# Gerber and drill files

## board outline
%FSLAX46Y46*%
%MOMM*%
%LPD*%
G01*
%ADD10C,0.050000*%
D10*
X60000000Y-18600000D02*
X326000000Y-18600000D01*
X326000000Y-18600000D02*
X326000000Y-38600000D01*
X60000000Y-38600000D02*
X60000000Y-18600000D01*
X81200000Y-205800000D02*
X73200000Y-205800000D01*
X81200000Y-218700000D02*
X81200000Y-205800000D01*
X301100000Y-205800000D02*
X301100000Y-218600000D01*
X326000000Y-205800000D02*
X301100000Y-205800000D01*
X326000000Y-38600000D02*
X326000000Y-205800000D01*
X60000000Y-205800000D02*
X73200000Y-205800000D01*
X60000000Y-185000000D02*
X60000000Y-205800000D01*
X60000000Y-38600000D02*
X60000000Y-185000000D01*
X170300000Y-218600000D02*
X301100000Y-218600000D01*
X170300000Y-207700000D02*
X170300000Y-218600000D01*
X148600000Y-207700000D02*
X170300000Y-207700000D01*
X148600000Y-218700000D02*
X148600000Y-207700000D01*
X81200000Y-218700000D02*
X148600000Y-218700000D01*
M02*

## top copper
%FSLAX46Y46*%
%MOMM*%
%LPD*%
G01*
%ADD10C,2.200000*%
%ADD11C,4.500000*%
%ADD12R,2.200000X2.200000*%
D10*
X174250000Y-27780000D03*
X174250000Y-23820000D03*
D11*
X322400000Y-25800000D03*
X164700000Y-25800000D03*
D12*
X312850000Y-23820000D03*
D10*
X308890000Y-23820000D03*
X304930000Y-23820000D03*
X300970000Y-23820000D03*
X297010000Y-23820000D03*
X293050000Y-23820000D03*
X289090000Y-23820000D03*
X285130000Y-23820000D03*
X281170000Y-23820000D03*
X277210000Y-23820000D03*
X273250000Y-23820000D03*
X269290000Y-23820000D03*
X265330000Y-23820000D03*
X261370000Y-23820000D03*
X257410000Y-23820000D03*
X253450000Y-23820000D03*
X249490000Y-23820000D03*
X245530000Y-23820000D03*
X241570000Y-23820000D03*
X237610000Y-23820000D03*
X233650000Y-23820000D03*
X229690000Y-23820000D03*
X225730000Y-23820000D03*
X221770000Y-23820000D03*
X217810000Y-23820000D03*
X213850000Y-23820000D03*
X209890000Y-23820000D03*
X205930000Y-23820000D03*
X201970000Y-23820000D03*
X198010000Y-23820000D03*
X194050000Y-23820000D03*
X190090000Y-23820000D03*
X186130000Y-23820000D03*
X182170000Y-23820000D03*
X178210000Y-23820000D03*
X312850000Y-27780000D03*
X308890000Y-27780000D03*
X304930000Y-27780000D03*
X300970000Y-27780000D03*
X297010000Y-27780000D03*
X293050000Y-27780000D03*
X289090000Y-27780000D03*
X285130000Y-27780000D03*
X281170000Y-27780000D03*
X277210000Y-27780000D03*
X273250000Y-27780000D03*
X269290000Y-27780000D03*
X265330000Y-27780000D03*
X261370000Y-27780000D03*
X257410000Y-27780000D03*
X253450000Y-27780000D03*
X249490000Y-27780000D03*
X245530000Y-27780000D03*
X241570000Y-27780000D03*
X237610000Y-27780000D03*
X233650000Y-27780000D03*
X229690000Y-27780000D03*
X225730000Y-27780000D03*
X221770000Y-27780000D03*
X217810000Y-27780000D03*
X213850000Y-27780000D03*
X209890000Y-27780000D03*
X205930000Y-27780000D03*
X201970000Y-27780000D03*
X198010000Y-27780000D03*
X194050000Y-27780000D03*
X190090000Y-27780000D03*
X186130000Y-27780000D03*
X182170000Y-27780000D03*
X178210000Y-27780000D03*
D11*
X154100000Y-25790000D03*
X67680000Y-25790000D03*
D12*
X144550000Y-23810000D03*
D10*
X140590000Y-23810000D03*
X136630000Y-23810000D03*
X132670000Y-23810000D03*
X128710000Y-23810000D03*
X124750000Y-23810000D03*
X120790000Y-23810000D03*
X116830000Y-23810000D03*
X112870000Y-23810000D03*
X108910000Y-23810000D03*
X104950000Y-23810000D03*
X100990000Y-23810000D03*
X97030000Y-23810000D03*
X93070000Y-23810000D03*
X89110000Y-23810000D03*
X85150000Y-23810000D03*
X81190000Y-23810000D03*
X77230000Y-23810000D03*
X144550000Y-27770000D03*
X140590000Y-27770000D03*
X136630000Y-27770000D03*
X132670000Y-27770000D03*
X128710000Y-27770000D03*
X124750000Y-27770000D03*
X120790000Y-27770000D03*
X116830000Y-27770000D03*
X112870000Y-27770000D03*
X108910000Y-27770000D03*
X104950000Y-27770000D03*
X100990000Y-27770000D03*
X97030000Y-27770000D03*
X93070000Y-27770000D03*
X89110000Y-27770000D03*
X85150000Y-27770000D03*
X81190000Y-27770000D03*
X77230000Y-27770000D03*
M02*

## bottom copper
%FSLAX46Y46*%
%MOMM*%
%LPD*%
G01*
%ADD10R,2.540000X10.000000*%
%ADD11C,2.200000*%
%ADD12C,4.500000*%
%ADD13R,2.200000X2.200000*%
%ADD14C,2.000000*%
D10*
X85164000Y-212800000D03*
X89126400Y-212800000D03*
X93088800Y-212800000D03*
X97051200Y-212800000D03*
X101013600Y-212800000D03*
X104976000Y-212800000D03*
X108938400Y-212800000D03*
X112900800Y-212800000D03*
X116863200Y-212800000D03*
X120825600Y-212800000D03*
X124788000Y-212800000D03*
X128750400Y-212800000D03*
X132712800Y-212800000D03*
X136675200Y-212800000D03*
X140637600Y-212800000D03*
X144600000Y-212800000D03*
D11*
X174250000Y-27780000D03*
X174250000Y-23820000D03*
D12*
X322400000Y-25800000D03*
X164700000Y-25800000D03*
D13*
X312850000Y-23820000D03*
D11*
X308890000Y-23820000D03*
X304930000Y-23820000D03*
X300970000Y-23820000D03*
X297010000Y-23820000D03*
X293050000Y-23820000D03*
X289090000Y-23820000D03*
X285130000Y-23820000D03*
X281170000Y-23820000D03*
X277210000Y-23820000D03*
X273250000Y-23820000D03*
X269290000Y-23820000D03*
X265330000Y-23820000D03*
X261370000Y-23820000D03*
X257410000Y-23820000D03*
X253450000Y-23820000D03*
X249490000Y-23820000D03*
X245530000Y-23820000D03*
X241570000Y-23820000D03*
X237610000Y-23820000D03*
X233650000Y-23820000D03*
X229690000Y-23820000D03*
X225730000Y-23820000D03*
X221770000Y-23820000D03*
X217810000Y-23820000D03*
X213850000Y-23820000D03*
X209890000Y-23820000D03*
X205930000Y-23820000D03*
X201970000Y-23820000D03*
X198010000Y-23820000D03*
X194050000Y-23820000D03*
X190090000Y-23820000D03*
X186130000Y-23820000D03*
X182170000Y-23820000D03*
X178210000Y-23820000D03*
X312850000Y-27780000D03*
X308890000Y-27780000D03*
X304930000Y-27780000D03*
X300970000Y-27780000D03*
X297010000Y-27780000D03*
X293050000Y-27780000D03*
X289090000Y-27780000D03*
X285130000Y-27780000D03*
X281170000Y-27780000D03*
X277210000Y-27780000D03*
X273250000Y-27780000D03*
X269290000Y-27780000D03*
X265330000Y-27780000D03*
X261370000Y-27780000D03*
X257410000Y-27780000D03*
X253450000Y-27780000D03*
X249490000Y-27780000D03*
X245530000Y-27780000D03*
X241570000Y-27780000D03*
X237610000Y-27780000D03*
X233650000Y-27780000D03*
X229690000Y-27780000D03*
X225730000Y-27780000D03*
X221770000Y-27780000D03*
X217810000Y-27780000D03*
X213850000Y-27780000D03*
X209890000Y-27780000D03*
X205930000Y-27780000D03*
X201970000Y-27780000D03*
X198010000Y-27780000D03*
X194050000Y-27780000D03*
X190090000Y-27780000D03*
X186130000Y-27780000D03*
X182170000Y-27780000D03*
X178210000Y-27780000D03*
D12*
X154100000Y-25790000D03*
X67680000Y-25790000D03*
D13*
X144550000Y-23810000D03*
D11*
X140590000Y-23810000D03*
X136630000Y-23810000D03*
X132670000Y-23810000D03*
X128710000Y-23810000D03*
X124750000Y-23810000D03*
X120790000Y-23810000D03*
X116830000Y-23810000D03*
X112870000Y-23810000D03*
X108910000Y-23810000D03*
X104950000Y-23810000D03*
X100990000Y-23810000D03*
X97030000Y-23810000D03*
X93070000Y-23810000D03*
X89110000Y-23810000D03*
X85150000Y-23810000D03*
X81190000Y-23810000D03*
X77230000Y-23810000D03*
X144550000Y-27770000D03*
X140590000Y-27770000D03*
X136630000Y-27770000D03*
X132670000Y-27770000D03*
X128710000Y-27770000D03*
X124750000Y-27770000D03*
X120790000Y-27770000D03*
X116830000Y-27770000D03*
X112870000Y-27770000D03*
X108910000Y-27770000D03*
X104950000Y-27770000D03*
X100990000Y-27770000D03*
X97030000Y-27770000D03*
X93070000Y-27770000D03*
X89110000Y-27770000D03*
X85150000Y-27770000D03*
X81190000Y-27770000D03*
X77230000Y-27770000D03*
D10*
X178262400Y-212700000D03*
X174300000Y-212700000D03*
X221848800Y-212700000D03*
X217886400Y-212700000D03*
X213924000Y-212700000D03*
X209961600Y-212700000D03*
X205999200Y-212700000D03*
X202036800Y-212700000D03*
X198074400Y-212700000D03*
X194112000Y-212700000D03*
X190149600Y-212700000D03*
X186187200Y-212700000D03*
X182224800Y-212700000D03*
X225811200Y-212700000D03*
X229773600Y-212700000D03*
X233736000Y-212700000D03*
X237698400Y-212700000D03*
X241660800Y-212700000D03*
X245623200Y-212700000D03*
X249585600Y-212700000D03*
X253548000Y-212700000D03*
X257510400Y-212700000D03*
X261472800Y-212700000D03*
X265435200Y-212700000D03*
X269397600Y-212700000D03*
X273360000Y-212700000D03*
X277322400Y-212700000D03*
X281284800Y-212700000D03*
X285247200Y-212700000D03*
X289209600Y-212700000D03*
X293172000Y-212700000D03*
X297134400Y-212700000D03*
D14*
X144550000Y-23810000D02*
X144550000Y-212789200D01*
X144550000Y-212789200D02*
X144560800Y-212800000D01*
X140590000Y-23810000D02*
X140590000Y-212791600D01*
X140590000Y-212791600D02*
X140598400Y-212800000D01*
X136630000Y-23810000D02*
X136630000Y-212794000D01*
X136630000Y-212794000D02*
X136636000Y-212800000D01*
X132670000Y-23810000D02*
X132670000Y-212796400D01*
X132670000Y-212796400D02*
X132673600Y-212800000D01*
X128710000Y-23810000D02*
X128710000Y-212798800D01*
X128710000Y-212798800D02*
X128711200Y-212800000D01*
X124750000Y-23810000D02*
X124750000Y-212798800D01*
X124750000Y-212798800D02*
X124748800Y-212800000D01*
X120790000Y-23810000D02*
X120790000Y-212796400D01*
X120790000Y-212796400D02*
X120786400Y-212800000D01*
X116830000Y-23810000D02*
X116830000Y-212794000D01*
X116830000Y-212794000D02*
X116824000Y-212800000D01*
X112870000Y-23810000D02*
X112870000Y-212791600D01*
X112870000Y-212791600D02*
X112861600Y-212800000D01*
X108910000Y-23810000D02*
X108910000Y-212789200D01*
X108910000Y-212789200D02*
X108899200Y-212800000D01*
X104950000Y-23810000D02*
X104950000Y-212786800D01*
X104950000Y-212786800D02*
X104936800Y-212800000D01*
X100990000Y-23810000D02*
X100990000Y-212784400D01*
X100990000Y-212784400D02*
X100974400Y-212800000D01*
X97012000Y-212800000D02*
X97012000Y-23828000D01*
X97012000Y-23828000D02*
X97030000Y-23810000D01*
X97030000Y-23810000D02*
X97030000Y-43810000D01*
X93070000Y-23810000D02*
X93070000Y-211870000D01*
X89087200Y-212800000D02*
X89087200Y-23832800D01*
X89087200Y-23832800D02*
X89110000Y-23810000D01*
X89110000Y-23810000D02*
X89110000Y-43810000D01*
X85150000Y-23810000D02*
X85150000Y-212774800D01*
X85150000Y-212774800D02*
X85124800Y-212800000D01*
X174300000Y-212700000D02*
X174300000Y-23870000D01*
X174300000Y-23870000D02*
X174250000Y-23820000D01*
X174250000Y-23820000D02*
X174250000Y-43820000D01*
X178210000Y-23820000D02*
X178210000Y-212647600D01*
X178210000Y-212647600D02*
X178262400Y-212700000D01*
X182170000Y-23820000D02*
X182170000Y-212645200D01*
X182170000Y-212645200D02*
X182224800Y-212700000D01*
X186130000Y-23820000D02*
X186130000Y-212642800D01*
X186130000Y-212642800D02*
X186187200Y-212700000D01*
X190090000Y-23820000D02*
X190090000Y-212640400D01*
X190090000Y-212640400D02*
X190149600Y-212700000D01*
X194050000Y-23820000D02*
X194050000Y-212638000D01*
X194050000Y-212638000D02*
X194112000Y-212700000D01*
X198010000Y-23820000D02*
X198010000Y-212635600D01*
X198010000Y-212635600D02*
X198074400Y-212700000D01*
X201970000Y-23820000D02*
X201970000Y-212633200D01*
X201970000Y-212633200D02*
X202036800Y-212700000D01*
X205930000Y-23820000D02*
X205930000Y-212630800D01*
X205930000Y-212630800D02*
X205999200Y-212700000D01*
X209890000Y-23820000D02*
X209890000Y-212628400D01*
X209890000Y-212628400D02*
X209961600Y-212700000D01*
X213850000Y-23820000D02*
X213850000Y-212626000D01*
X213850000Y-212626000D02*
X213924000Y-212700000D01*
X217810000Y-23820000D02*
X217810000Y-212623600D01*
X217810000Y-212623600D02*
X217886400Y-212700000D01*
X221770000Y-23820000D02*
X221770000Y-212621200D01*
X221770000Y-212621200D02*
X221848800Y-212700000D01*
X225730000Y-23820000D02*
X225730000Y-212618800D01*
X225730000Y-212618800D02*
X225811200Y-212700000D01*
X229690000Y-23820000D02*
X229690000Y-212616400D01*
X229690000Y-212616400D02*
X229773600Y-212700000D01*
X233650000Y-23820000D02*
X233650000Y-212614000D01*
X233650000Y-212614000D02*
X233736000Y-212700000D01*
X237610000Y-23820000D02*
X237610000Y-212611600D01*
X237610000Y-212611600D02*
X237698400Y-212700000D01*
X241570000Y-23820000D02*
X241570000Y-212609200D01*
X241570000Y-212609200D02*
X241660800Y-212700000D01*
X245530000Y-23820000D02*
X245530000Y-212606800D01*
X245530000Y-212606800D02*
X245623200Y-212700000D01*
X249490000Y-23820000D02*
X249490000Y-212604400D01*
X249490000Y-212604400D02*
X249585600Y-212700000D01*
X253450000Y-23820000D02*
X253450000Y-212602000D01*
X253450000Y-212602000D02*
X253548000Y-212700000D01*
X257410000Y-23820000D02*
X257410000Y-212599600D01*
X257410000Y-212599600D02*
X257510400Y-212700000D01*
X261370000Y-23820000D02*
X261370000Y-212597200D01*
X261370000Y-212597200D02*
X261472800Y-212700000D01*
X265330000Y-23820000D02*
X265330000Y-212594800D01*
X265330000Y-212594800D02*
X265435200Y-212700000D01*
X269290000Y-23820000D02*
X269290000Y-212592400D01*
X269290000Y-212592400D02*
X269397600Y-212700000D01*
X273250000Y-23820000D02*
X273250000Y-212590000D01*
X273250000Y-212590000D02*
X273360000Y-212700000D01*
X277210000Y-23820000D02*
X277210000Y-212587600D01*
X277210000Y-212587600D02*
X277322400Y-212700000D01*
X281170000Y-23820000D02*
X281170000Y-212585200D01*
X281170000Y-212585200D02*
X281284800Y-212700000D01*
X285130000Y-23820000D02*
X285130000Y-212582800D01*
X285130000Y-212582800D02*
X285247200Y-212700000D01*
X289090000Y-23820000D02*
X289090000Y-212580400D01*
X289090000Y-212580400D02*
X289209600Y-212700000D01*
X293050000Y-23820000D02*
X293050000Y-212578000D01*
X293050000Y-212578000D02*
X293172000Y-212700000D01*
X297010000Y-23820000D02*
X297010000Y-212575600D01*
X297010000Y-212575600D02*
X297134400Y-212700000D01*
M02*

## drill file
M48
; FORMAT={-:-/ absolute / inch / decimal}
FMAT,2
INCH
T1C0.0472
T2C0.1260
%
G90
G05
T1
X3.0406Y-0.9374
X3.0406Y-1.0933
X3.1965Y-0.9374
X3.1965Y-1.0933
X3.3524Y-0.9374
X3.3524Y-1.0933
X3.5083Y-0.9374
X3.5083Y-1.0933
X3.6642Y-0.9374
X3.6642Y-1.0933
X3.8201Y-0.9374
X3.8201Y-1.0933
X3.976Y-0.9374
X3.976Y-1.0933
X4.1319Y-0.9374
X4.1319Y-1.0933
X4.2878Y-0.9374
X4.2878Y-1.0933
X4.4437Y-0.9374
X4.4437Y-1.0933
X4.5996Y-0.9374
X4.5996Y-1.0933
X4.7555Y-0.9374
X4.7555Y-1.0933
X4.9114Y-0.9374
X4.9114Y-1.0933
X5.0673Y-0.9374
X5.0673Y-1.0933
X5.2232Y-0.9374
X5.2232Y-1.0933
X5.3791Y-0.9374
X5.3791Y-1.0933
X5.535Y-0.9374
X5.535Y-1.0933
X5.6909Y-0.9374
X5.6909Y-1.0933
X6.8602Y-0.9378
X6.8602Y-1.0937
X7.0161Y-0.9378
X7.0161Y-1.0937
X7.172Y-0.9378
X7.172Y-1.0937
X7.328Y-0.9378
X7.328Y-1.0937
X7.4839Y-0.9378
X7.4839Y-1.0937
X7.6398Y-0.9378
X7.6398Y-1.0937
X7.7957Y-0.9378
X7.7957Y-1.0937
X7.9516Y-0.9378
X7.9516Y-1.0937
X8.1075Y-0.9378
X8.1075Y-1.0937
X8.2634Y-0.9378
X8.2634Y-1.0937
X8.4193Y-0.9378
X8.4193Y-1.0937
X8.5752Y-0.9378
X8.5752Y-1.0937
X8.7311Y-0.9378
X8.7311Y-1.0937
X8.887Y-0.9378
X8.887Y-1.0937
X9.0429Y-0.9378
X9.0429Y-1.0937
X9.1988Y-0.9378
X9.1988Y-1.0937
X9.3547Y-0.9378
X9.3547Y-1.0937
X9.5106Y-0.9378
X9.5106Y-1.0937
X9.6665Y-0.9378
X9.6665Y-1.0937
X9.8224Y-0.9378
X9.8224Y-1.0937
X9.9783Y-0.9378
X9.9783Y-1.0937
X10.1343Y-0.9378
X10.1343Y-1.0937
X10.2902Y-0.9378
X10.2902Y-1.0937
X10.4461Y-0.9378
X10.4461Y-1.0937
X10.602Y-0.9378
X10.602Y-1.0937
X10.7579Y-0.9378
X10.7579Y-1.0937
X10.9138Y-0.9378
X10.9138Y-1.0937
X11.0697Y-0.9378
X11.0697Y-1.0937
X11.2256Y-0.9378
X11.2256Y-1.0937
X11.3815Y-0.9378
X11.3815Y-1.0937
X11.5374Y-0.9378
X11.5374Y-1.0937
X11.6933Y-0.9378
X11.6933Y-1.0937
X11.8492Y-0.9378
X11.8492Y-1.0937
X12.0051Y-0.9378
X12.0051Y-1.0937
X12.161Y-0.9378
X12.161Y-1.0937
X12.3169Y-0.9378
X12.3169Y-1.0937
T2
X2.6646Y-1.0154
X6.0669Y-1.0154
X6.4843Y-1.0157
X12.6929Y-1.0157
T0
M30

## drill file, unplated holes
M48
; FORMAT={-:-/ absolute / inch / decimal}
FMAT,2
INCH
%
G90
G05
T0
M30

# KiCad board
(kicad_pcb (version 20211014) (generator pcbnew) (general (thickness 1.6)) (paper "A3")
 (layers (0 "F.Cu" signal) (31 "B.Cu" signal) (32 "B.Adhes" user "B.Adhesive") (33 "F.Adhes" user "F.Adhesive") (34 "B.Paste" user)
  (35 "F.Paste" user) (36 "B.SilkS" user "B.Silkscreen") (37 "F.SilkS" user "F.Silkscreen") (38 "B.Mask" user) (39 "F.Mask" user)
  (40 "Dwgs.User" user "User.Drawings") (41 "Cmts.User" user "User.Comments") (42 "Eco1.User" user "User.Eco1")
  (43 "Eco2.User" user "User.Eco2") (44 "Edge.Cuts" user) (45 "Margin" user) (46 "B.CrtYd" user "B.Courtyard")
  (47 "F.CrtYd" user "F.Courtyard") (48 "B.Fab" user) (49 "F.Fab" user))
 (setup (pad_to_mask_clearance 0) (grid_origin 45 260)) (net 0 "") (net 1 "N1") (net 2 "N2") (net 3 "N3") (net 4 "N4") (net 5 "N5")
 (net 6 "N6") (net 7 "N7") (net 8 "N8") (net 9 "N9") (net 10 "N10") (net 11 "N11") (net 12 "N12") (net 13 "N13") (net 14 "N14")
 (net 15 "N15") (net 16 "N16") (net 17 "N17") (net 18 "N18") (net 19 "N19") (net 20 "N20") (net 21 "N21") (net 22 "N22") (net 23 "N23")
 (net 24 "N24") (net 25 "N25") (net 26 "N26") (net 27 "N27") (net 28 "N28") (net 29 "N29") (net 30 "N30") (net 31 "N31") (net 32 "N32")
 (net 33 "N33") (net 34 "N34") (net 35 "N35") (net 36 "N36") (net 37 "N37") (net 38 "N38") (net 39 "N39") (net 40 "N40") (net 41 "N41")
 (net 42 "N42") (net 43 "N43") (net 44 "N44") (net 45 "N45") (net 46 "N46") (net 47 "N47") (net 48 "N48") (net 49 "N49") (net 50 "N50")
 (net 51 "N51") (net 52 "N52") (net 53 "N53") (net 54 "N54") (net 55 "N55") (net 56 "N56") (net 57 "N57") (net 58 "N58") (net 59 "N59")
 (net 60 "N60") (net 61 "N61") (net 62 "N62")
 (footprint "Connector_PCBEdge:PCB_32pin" (layer "F.Cu") (at 170.278 218.582)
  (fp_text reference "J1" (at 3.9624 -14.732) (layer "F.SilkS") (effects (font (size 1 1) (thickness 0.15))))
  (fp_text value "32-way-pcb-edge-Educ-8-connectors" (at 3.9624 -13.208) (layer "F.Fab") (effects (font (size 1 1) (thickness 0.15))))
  (pad "1" connect rect locked (at 126.8564 -5.882) (size 2.54 10) (layers "B.Cu" "B.Mask") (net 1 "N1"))
  (pad "2" connect rect locked (at 122.894 -5.882) (size 2.54 10) (layers "B.Cu" "B.Mask") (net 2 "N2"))
  (pad "3" connect rect locked (at 118.9316 -5.882) (size 2.54 10) (layers "B.Cu" "B.Mask") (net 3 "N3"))
  (pad "4" connect rect locked (at 114.9692 -5.882) (size 2.54 10) (layers "B.Cu" "B.Mask") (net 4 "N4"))
  (pad "5" connect rect locked (at 111.0068 -5.882) (size 2.54 10) (layers "B.Cu" "B.Mask") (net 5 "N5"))
  (pad "6" connect rect locked (at 107.0444 -5.882) (size 2.54 10) (layers "B.Cu" "B.Mask") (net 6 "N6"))
  (pad "7" connect rect locked (at 103.082 -5.882) (size 2.54 10) (layers "B.Cu" "B.Mask") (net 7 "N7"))
  (pad "8" connect rect locked (at 99.1196 -5.882) (size 2.54 10) (layers "B.Cu" "B.Mask") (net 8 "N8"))
  (pad "9" connect rect locked (at 95.1572 -5.882) (size 2.54 10) (layers "B.Cu" "B.Mask") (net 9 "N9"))
  (pad "10" connect rect locked (at 91.1948 -5.882) (size 2.54 10) (layers "B.Cu" "B.Mask") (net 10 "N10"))
  (pad "11" connect rect locked (at 87.2324 -5.882) (size 2.54 10) (layers "B.Cu" "B.Mask") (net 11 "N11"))
  (pad "12" connect rect locked (at 83.27 -5.882) (size 2.54 10) (layers "B.Cu" "B.Mask") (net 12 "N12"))
  (pad "13" connect rect locked (at 79.3076 -5.882) (size 2.54 10) (layers "B.Cu" "B.Mask") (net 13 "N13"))
  (pad "14" connect rect locked (at 75.3452 -5.882) (size 2.54 10) (layers "B.Cu" "B.Mask") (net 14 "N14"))
  (pad "15" connect rect locked (at 71.3828 -5.882) (size 2.54 10) (layers "B.Cu" "B.Mask") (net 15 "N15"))
  (pad "16" connect rect locked (at 67.4204 -5.882) (size 2.54 10) (layers "B.Cu" "B.Mask") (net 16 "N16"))
  (pad "17" connect rect locked (at 63.458 -5.882) (size 2.54 10) (layers "B.Cu" "B.Mask") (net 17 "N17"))
  (pad "18" connect rect locked (at 59.4956 -5.882) (size 2.54 10) (layers "B.Cu" "B.Mask") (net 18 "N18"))
  (pad "19" connect rect locked (at 55.5332 -5.882) (size 2.54 10) (layers "B.Cu" "B.Mask") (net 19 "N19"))
  (pad "20" connect rect locked (at 51.5708 -5.882) (size 2.54 10) (layers "B.Cu" "B.Mask") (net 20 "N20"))
  (pad "21" connect rect locked (at 47.6084 -5.882) (size 2.54 10) (layers "B.Cu" "B.Mask") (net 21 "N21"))
  (pad "22" connect rect locked (at 43.646 -5.882) (size 2.54 10) (layers "B.Cu" "B.Mask") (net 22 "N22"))
  (pad "23" connect rect locked (at 39.6836 -5.882) (size 2.54 10) (layers "B.Cu" "B.Mask") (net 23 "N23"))
  (pad "24" connect rect locked (at 35.7212 -5.882) (size 2.54 10) (layers "B.Cu" "B.Mask") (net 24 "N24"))
  (pad "25" connect rect locked (at 31.7588 -5.882) (size 2.54 10) (layers "B.Cu" "B.Mask") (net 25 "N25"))
  (pad "26" connect rect locked (at 27.7964 -5.882) (size 2.54 10) (layers "B.Cu" "B.Mask") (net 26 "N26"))
  (pad "27" connect rect locked (at 23.834 -5.882) (size 2.54 10) (layers "B.Cu" "B.Mask") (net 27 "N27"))
  (pad "28" connect rect locked (at 19.8716 -5.882) (size 2.54 10) (layers "B.Cu" "B.Mask") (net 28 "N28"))
  (pad "29" connect rect locked (at 15.9092 -5.882) (size 2.54 10) (layers "B.Cu" "B.Mask") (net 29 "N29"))
  (pad "30" connect rect locked (at 11.9468 -5.882) (size 2.54 10) (layers "B.Cu" "B.Mask") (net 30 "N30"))
  (pad "31" connect rect locked (at 7.9844 -5.882) (size 2.54 10) (layers "B.Cu" "B.Mask") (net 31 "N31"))
  (pad "32" connect rect locked (at 4.022 -5.882) (size 2.54 10) (layers "B.Cu" "B.Mask") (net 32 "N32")))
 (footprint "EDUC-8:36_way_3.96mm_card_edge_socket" (layer "F.Cu") (at 154.1 25.79 180)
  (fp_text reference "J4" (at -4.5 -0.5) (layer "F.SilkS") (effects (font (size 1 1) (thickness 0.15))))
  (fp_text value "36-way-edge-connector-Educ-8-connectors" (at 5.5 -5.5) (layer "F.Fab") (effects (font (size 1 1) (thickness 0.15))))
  (pad "1" thru_hole rect locked (at 9.55 1.98 180) (size 2.2 2.2) (drill 1.2) (layers *.Cu *.Mask) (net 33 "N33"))
  (pad "2" thru_hole circle locked (at 13.51 1.98 180) (size 2.2 2.2) (drill 1.2) (layers *.Cu *.Mask) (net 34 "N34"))
  (pad "3" thru_hole circle locked (at 17.47 1.98 180) (size 2.2 2.2) (drill 1.2) (layers *.Cu *.Mask) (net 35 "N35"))
  (pad "4" thru_hole circle locked (at 21.43 1.98 180) (size 2.2 2.2) (drill 1.2) (layers *.Cu *.Mask) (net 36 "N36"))
  (pad "5" thru_hole circle locked (at 25.39 1.98 180) (size 2.2 2.2) (drill 1.2) (layers *.Cu *.Mask) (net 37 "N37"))
  (pad "6" thru_hole circle locked (at 29.35 1.98 180) (size 2.2 2.2) (drill 1.2) (layers *.Cu *.Mask) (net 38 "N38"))
  (pad "7" thru_hole circle locked (at 33.31 1.98 180) (size 2.2 2.2) (drill 1.2) (layers *.Cu *.Mask) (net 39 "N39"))
  (pad "8" thru_hole circle locked (at 37.27 1.98 180) (size 2.2 2.2) (drill 1.2) (layers *.Cu *.Mask) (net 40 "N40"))
  (pad "9" thru_hole circle locked (at 41.23 1.98 180) (size 2.2 2.2) (drill 1.2) (layers *.Cu *.Mask) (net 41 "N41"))
  (pad "10" thru_hole circle locked (at 45.19 1.98 180) (size 2.2 2.2) (drill 1.2) (layers *.Cu *.Mask) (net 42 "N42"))
  (pad "11" thru_hole circle locked (at 49.15 1.98 180) (size 2.2 2.2) (drill 1.2) (layers *.Cu *.Mask) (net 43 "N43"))
  (pad "12" thru_hole circle locked (at 53.11 1.98 180) (size 2.2 2.2) (drill 1.2) (layers *.Cu *.Mask) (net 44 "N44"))
  (pad "13" thru_hole circle locked (at 57.07 1.98 180) (size 2.2 2.2) (drill 1.2) (layers *.Cu *.Mask) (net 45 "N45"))
  (pad "14" thru_hole circle locked (at 61.03 1.98 180) (size 2.2 2.2) (drill 1.2) (layers *.Cu *.Mask) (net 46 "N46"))
  (pad "15" thru_hole circle locked (at 64.99 1.98 180) (size 2.2 2.2) (drill 1.2) (layers *.Cu *.Mask) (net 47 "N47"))
  (pad "16" thru_hole circle locked (at 68.95 1.98 180) (size 2.2 2.2) (drill 1.2) (layers *.Cu *.Mask) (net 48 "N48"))
  (pad "17" thru_hole circle locked (at 72.91 1.98 180) (size 2.2 2.2) (drill 1.2) (layers *.Cu *.Mask) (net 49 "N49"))
  (pad "18" thru_hole circle locked (at 76.87 1.98 180) (size 2.2 2.2) (drill 1.2) (layers *.Cu *.Mask) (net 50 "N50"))
  (pad "A" thru_hole circle locked (at 9.55 -1.98 180) (size 2.2 2.2) (drill 1.2) (layers *.Cu *.Mask) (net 33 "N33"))
  (pad "B" thru_hole circle locked (at 13.51 -1.98 180) (size 2.2 2.2) (drill 1.2) (layers *.Cu *.Mask) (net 34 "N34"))
  (pad "C" thru_hole circle locked (at 17.47 -1.98 180) (size 2.2 2.2) (drill 1.2) (layers *.Cu *.Mask) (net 35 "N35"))
  (pad "D" thru_hole circle locked (at 21.43 -1.98 180) (size 2.2 2.2) (drill 1.2) (layers *.Cu *.Mask) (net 36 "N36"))
  (pad "E" thru_hole circle locked (at 25.39 -1.98 180) (size 2.2 2.2) (drill 1.2) (layers *.Cu *.Mask) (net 37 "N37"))
  (pad "F" thru_hole circle locked (at 29.35 -1.98 180) (size 2.2 2.2) (drill 1.2) (layers *.Cu *.Mask) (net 38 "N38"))
  (pad "G" thru_hole circle locked (at 33.31 -1.98 180) (size 2.2 2.2) (drill 1.2) (layers *.Cu *.Mask) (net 39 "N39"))
  (pad "H" thru_hole circle locked (at 37.27 -1.98 180) (size 2.2 2.2) (drill 1.2) (layers *.Cu *.Mask) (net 40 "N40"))
  (pad "H1" thru_hole circle locked (at 0 0 180) (size 4.5 4.5) (drill 3.2) (layers *.Cu *.Mask) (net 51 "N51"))
  (pad "H2" thru_hole circle locked (at 86.42 0 180) (size 4.5 4.5) (drill 3.2) (layers *.Cu *.Mask) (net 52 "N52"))
  (pad "J" thru_hole circle locked (at 41.23 -1.98 180) (size 2.2 2.2) (drill 1.2) (layers *.Cu *.Mask) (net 41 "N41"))
  (pad "K" thru_hole circle locked (at 45.19 -1.98 180) (size 2.2 2.2) (drill 1.2) (layers *.Cu *.Mask) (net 42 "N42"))
  (pad "L" thru_hole circle locked (at 49.15 -1.98 180) (size 2.2 2.2) (drill 1.2) (layers *.Cu *.Mask) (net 43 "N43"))
  (pad "M" thru_hole circle locked (at 53.11 -1.98 180) (size 2.2 2.2) (drill 1.2) (layers *.Cu *.Mask) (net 44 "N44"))
  (pad "N" thru_hole circle locked (at 57.07 -1.98 180) (size 2.2 2.2) (drill 1.2) (layers *.Cu *.Mask) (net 45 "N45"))
  (pad "P" thru_hole circle locked (at 61.03 -1.98 180) (size 2.2 2.2) (drill 1.2) (layers *.Cu *.Mask) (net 46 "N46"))
  (pad "Q" thru_hole circle locked (at 64.99 -1.98 180) (size 2.2 2.2) (drill 1.2) (layers *.Cu *.Mask) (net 47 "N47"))
  (pad "R" thru_hole circle locked (at 68.95 -1.98 180) (size 2.2 2.2) (drill 1.2) (layers *.Cu *.Mask) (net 48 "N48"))
  (pad "S" thru_hole circle locked (at 72.91 -1.98 180) (size 2.2 2.2) (drill 1.2) (layers *.Cu *.Mask) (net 49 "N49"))
  (pad "T" thru_hole circle locked (at 76.87 -1.98 180) (size 2.2 2.2) (drill 1.2) (layers *.Cu *.Mask) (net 50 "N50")))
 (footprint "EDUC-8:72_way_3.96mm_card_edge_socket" (layer "F.Cu") (at 322.4 25.8 180)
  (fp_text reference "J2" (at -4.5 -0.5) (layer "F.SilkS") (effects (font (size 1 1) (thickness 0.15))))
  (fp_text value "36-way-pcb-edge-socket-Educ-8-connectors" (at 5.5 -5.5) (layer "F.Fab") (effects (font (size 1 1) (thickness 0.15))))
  (pad "1" thru_hole rect locked (at 9.55 1.98 180) (size 2.2 2.2) (drill 1.2) (layers *.Cu *.Mask) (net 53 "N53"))
  (pad "2" thru_hole circle locked (at 13.51 1.98 180) (size 2.2 2.2) (drill 1.2) (layers *.Cu *.Mask) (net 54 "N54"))
  (pad "3" thru_hole circle locked (at 17.47 1.98 180) (size 2.2 2.2) (drill 1.2) (layers *.Cu *.Mask) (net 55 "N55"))
  (pad "4" thru_hole circle locked (at 21.43 1.98 180) (size 2.2 2.2) (drill 1.2) (layers *.Cu *.Mask) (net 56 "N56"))
  (pad "5" thru_hole circle locked (at 25.39 1.98 180) (size 2.2 2.2) (drill 1.2) (layers *.Cu *.Mask) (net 1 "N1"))
  (pad "6" thru_hole circle locked (at 29.35 1.98 180) (size 2.2 2.2) (drill 1.2) (layers *.Cu *.Mask) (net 2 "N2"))
  (pad "7" thru_hole circle locked (at 33.31 1.98 180) (size 2.2 2.2) (drill 1.2) (layers *.Cu *.Mask) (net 3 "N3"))
  (pad "8" thru_hole circle locked (at 37.27 1.98 180) (size 2.2 2.2) (drill 1.2) (layers *.Cu *.Mask) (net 4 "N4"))
  (pad "9" thru_hole circle locked (at 41.23 1.98 180) (size 2.2 2.2) (drill 1.2) (layers *.Cu *.Mask) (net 5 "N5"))
  (pad "10" thru_hole circle locked (at 45.19 1.98 180) (size 2.2 2.2) (drill 1.2) (layers *.Cu *.Mask) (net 6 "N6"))
  (pad "11" thru_hole circle locked (at 49.15 1.98 180) (size 2.2 2.2) (drill 1.2) (layers *.Cu *.Mask) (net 7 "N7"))
  (pad "12" thru_hole circle locked (at 53.11 1.98 180) (size 2.2 2.2) (drill 1.2) (layers *.Cu *.Mask) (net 8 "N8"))
  (pad "13" thru_hole circle locked (at 57.07 1.98 180) (size 2.2 2.2) (drill 1.2) (layers *.Cu *.Mask) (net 9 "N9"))
  (pad "14" thru_hole circle locked (at 61.03 1.98 180) (size 2.2 2.2) (drill 1.2) (layers *.Cu *.Mask) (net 10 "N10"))
  (pad "15" thru_hole circle locked (at 64.99 1.98 180) (size 2.2 2.2) (drill 1.2) (layers *.Cu *.Mask) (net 11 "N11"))
  (pad "16" thru_hole circle locked (at 68.95 1.98 180) (size 2.2 2.2) (drill 1.2) (layers *.Cu *.Mask) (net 12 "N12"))
  (pad "17" thru_hole circle locked (at 72.91 1.98 180) (size 2.2 2.2) (drill 1.2) (layers *.Cu *.Mask) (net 13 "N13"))
  (pad "18" thru_hole circle locked (at 76.87 1.98 180) (size 2.2 2.2) (drill 1.2) (layers *.Cu *.Mask) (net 14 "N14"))
  (pad "19" thru_hole circle locked (at 80.83 1.98 180) (size 2.2 2.2) (drill 1.2) (layers *.Cu *.Mask) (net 15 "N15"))
  (pad "20" thru_hole circle locked (at 84.79 1.98 180) (size 2.2 2.2) (drill 1.2) (layers *.Cu *.Mask) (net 16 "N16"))
  (pad "21" thru_hole circle locked (at 88.75 1.98 180) (size 2.2 2.2) (drill 1.2) (layers *.Cu *.Mask) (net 17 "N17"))
  (pad "22" thru_hole circle locked (at 92.71 1.98 180) (size 2.2 2.2) (drill 1.2) (layers *.Cu *.Mask) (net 18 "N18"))
  (pad "23" thru_hole circle locked (at 96.67 1.98 180) (size 2.2 2.2) (drill 1.2) (layers *.Cu *.Mask) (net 19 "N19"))
  (pad "24" thru_hole circle locked (at 100.63 1.98 180) (size 2.2 2.2) (drill 1.2) (layers *.Cu *.Mask) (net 20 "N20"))
  (pad "25" thru_hole circle locked (at 104.59 1.98 180) (size 2.2 2.2) (drill 1.2) (layers *.Cu *.Mask) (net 21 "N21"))
  (pad "26" thru_hole circle locked (at 108.55 1.98 180) (size 2.2 2.2) (drill 1.2) (layers *.Cu *.Mask) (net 22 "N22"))
  (pad "27" thru_hole circle locked (at 112.51 1.98 180) (size 2.2 2.2) (drill 1.2) (layers *.Cu *.Mask) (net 23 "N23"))
  (pad "28" thru_hole circle locked (at 116.47 1.98 180) (size 2.2 2.2) (drill 1.2) (layers *.Cu *.Mask) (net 24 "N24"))
  (pad "29" thru_hole circle locked (at 120.43 1.98 180) (size 2.2 2.2) (drill 1.2) (layers *.Cu *.Mask) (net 25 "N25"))
  (pad "30" thru_hole circle locked (at 124.39 1.98 180) (size 2.2 2.2) (drill 1.2) (layers *.Cu *.Mask) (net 26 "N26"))
  (pad "31" thru_hole circle locked (at 128.35 1.98 180) (size 2.2 2.2) (drill 1.2) (layers *.Cu *.Mask) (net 27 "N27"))
  (pad "32" thru_hole circle locked (at 132.31 1.98 180) (size 2.2 2.2) (drill 1.2) (layers *.Cu *.Mask) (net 28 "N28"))
  (pad "33" thru_hole circle locked (at 136.27 1.98 180) (size 2.2 2.2) (drill 1.2) (layers *.Cu *.Mask) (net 29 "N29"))
  (pad "34" thru_hole circle locked (at 140.23 1.98 180) (size 2.2 2.2) (drill 1.2) (layers *.Cu *.Mask) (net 30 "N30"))
  (pad "35" thru_hole circle locked (at 144.19 1.98 180) (size 2.2 2.2) (drill 1.2) (layers *.Cu *.Mask) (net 31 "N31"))
  (pad "36" thru_hole circle locked (at 148.15 1.98 180) (size 2.2 2.2) (drill 1.2) (layers *.Cu *.Mask) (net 32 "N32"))
  (pad "A1" thru_hole circle locked (at 9.55 -1.98 180) (size 2.2 2.2) (drill 1.2) (layers *.Cu *.Mask) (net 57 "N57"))
  (pad "A2" thru_hole circle locked (at 13.51 -1.98 180) (size 2.2 2.2) (drill 1.2) (layers *.Cu *.Mask) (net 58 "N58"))
  (pad "A3" thru_hole circle locked (at 17.47 -1.98 180) (size 2.2 2.2) (drill 1.2) (layers *.Cu *.Mask) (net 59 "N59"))
  (pad "A4" thru_hole circle locked (at 21.43 -1.98 180) (size 2.2 2.2) (drill 1.2) (layers *.Cu *.Mask) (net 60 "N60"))
  (pad "A5" thru_hole circle locked (at 25.39 -1.98 180) (size 2.2 2.2) (drill 1.2) (layers *.Cu *.Mask) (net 1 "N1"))
  (pad "A6" thru_hole circle locked (at 29.35 -1.98 180) (size 2.2 2.2) (drill 1.2) (layers *.Cu *.Mask) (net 2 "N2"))
  (pad "A7" thru_hole circle locked (at 33.31 -1.98 180) (size 2.2 2.2) (drill 1.2) (layers *.Cu *.Mask) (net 3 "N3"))
  (pad "A8" thru_hole circle locked (at 37.27 -1.98 180) (size 2.2 2.2) (drill 1.2) (layers *.Cu *.Mask) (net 4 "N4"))
  (pad "A9" thru_hole circle locked (at 41.23 -1.98 180) (size 2.2 2.2) (drill 1.2) (layers *.Cu *.Mask) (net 5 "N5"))
  (pad "A10" thru_hole circle locked (at 45.19 -1.98 180) (size 2.2 2.2) (drill 1.2) (layers *.Cu *.Mask) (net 6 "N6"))
  (pad "A11" thru_hole circle locked (at 49.15 -1.98 180) (size 2.2 2.2) (drill 1.2) (layers *.Cu *.Mask) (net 7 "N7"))
  (pad "A12" thru_hole circle locked (at 53.11 -1.98 180) (size 2.2 2.2) (drill 1.2) (layers *.Cu *.Mask) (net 8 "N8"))
  (pad "A13" thru_hole circle locked (at 57.07 -1.98 180) (size 2.2 2.2) (drill 1.2) (layers *.Cu *.Mask) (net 9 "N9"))
  (pad "A14" thru_hole circle locked (at 61.03 -1.98 180) (size 2.2 2.2) (drill 1.2) (layers *.Cu *.Mask) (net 10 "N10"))
  (pad "A15" thru_hole circle locked (at 64.99 -1.98 180) (size 2.2 2.2) (drill 1.2) (layers *.Cu *.Mask) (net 11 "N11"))
  (pad "A16" thru_hole circle locked (at 68.95 -1.98 180) (size 2.2 2.2) (drill 1.2) (layers *.Cu *.Mask) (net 12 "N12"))
  (pad "A17" thru_hole circle locked (at 72.91 -1.98 180) (size 2.2 2.2) (drill 1.2) (layers *.Cu *.Mask) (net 13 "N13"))
  (pad "A18" thru_hole circle locked (at 76.87 -1.98 180) (size 2.2 2.2) (drill 1.2) (layers *.Cu *.Mask) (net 14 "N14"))
  (pad "A19" thru_hole circle locked (at 80.83 -1.98 180) (size 2.2 2.2) (drill 1.2) (layers *.Cu *.Mask) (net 15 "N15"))
  (pad "A20" thru_hole circle locked (at 84.79 -1.98 180) (size 2.2 2.2) (drill 1.2) (layers *.Cu *.Mask) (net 16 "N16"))
  (pad "A21" thru_hole circle locked (at 88.75 -1.98 180) (size 2.2 2.2) (drill 1.2) (layers *.Cu *.Mask) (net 17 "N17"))
  (pad "A22" thru_hole circle locked (at 92.71 -1.98 180) (size 2.2 2.2) (drill 1.2) (layers *.Cu *.Mask) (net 18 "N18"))
  (pad "A23" thru_hole circle locked (at 96.67 -1.98 180) (size 2.2 2.2) (drill 1.2) (layers *.Cu *.Mask) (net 19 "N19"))
  (pad "A24" thru_hole circle locked (at 100.63 -1.98 180) (size 2.2 2.2) (drill 1.2) (layers *.Cu *.Mask) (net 20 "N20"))
  (pad "A25" thru_hole circle locked (at 104.59 -1.98 180) (size 2.2 2.2) (drill 1.2) (layers *.Cu *.Mask) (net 21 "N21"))
  (pad "A26" thru_hole circle locked (at 108.55 -1.98 180) (size 2.2 2.2) (drill 1.2) (layers *.Cu *.Mask) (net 22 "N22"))
  (pad "A27" thru_hole circle locked (at 112.51 -1.98 180) (size 2.2 2.2) (drill 1.2) (layers *.Cu *.Mask) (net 23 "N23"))
  (pad "A28" thru_hole circle locked (at 116.47 -1.98 180) (size 2.2 2.2) (drill 1.2) (layers *.Cu *.Mask) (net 24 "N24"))
  (pad "A29" thru_hole circle locked (at 120.43 -1.98 180) (size 2.2 2.2) (drill 1.2) (layers *.Cu *.Mask) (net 25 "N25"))
  (pad "A30" thru_hole circle locked (at 124.39 -1.98 180) (size 2.2 2.2) (drill 1.2) (layers *.Cu *.Mask) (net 26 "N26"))
  (pad "A31" thru_hole circle locked (at 128.35 -1.98 180) (size 2.2 2.2) (drill 1.2) (layers *.Cu *.Mask) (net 27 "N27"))
  (pad "A32" thru_hole circle locked (at 132.31 -1.98 180) (size 2.2 2.2) (drill 1.2) (layers *.Cu *.Mask) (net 28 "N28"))
  (pad "A33" thru_hole circle locked (at 136.27 -1.98 180) (size 2.2 2.2) (drill 1.2) (layers *.Cu *.Mask) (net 29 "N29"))
  (pad "A34" thru_hole circle locked (at 140.23 -1.98 180) (size 2.2 2.2) (drill 1.2) (layers *.Cu *.Mask) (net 30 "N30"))
  (pad "A35" thru_hole circle locked (at 144.19 -1.98 180) (size 2.2 2.2) (drill 1.2) (layers *.Cu *.Mask) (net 31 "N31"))
  (pad "A36" thru_hole circle locked (at 148.15 -1.98 180) (size 2.2 2.2) (drill 1.2) (layers *.Cu *.Mask) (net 32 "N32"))
  (pad "H1" thru_hole circle locked (at 0 0 180) (size 4.5 4.5) (drill 3.2) (layers *.Cu *.Mask) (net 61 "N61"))
  (pad "H2" thru_hole circle locked (at 157.7 0 180) (size 4.5 4.5) (drill 3.2) (layers *.Cu *.Mask) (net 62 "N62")))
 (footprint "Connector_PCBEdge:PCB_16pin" (layer "F.Cu") (at 81.1768 218.742)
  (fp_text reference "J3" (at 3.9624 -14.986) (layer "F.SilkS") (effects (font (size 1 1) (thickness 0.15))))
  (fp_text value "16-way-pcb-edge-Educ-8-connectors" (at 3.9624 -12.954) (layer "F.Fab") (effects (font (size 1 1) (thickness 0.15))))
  (pad "1" connect rect locked (at 63.4232 -5.942) (size 2.54 10) (layers "B.Cu" "B.Mask") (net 33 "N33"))
  (pad "2" connect rect locked (at 59.4608 -5.942) (size 2.54 10) (layers "B.Cu" "B.Mask") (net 34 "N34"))
  (pad "3" connect rect locked (at 55.4984 -5.942) (size 2.54 10) (layers "B.Cu" "B.Mask") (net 35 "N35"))
  (pad "4" connect rect locked (at 51.536 -5.942) (size 2.54 10) (layers "B.Cu" "B.Mask") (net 36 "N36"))
  (pad "5" connect rect locked (at 47.5736 -5.942) (size 2.54 10) (layers "B.Cu" "B.Mask") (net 37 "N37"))
  (pad "6" connect rect locked (at 43.6112 -5.942) (size 2.54 10) (layers "B.Cu" "B.Mask") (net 38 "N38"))
  (pad "7" connect rect locked (at 39.6488 -5.942) (size 2.54 10) (layers "B.Cu" "B.Mask") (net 39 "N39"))
  (pad "8" connect rect locked (at 35.6864 -5.942) (size 2.54 10) (layers "B.Cu" "B.Mask") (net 40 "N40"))
  (pad "9" connect rect locked (at 31.724 -5.942) (size 2.54 10) (layers "B.Cu" "B.Mask") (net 41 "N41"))
  (pad "10" connect rect locked (at 27.7616 -5.942) (size 2.54 10) (layers "B.Cu" "B.Mask") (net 42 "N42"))
  (pad "11" connect rect locked (at 23.7992 -5.942) (size 2.54 10) (layers "B.Cu" "B.Mask") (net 43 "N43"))
  (pad "12" connect rect locked (at 19.8368 -5.942) (size 2.54 10) (layers "B.Cu" "B.Mask") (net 44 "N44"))
  (pad "13" connect rect locked (at 15.8744 -5.942) (size 2.54 10) (layers "B.Cu" "B.Mask") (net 45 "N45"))
  (pad "14" connect rect locked (at 11.912 -5.942) (size 2.54 10) (layers "B.Cu" "B.Mask") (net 46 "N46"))
  (pad "15" connect rect locked (at 7.9496 -5.942) (size 2.54 10) (layers "B.Cu" "B.Mask") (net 47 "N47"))
  (pad "16" connect rect locked (at 3.9872 -5.942) (size 2.54 10) (layers "B.Cu" "B.Mask") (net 48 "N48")))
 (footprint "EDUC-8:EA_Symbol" (layer "F.Cu") (at 71.9 139.5 90)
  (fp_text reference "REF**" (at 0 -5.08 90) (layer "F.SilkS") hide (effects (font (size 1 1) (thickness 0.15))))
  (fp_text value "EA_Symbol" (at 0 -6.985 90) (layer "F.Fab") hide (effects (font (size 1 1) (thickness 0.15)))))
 (gr_line (start 170.3 218.6) (end 301.1 218.6) (layer "Edge.Cuts") (width 0.05))
 (gr_line (start 301.1 205.8) (end 301.1 218.6) (layer "Edge.Cuts") (width 0.05))
 (gr_line (start 81.2 205.8) (end 73.2 205.8) (layer "Edge.Cuts") (width 0.05))
 (gr_line (start 60 185) (end 60 205.8) (layer "Edge.Cuts") (width 0.05))
 (gr_line (start 148.6 218.7) (end 148.6 207.7) (layer "Edge.Cuts") (width 0.05))
 (gr_line (start 60 205.8) (end 73.2 205.8) (layer "Edge.Cuts") (width 0.05))
 (gr_line (start 170.3 207.7) (end 170.3 218.6) (layer "Edge.Cuts") (width 0.05))
 (gr_line (start 81.2 218.7) (end 81.2 205.8) (layer "Edge.Cuts") (width 0.05))
 (gr_line (start 60 38.6) (end 60 18.6) (layer "Edge.Cuts") (width 0.05))
 (gr_line (start 60 18.6) (end 326 18.6) (layer "Edge.Cuts") (width 0.05))
 (gr_line (start 326 38.6) (end 326 205.8) (layer "Edge.Cuts") (width 0.05))
 (gr_line (start 60 38.6) (end 60 185) (layer "Edge.Cuts") (width 0.05))
 (gr_line (start 326 205.8) (end 301.1 205.8) (layer "Edge.Cuts") (width 0.05))
 (gr_line (start 148.6 207.7) (end 170.3 207.7) (layer "Edge.Cuts") (width 0.05))
 (gr_line (start 81.2 218.7) (end 148.6 218.7) (layer "Edge.Cuts") (width 0.05))
 (gr_line (start 326 18.6) (end 326 38.6) (layer "Edge.Cuts") (width 0.05))
 (segment (start 178.21 23.82) (end 178.21 212.6476) (width 2) (layer "B.Cu") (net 31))
 (segment (start 178.21 212.6476) (end 178.2624 212.7) (width 2) (layer "B.Cu") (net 31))
 (segment (start 174.3 23.87) (end 174.25 23.82) (width 2) (layer "B.Cu") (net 32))
 (segment (start 174.3 212.7) (end 174.3 23.87) (width 2) (layer "B.Cu") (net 32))
 (segment (start 174.25 23.82) (end 174.25 43.82) (width 2) (layer "B.Cu") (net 32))
 (segment (start 221.77 23.82) (end 221.77 212.6212) (width 2) (layer "B.Cu") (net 20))
 (segment (start 221.77 212.6212) (end 221.8488 212.7) (width 2) (layer "B.Cu") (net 20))
 (segment (start 217.81 212.6236) (end 217.8864 212.7) (width 2) (layer "B.Cu") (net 21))
 (segment (start 217.81 23.82) (end 217.81 212.6236) (width 2) (layer "B.Cu") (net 21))
 (segment (start 213.85 23.82) (end 213.85 212.626) (width 2) (layer "B.Cu") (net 22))
 (segment (start 213.85 212.626) (end 213.924 212.7) (width 2) (layer "B.Cu") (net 22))
 (segment (start 209.89 212.6284) (end 209.9616 212.7) (width 2) (layer "B.Cu") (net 23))
 (segment (start 209.89 23.82) (end 209.89 212.6284) (width 2) (layer "B.Cu") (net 23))
 (segment (start 205.93 23.82) (end 205.93 212.6308) (width 2) (layer "B.Cu") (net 24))
 (segment (start 205.93 212.6308) (end 205.9992 212.7) (width 2) (layer "B.Cu") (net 24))
 (segment (start 201.97 23.82) (end 201.97 212.6332) (width 2) (layer "B.Cu") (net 25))
 (segment (start 201.97 212.6332) (end 202.0368 212.7) (width 2) (layer "B.Cu") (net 25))
 (segment (start 198.01 212.6356) (end 198.0744 212.7) (width 2) (layer "B.Cu") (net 26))
 (segment (start 198.01 23.82) (end 198.01 212.6356) (width 2) (layer "B.Cu") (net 26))
 (segment (start 194.05 212.638) (end 194.112 212.7) (width 2) (layer "B.Cu") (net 27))
 (segment (start 194.05 23.82) (end 194.05 212.638) (width 2) (layer "B.Cu") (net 27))
 (segment (start 190.09 212.6404) (end 190.1496 212.7) (width 2) (layer "B.Cu") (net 28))
 (segment (start 190.09 23.82) (end 190.09 212.6404) (width 2) (layer "B.Cu") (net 28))
 (segment (start 186.13 23.82) (end 186.13 212.6428) (width 2) (layer "B.Cu") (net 29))
 (segment (start 186.13 212.6428) (end 186.1872 212.7) (width 2) (layer "B.Cu") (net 29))
 (segment (start 182.17 23.82) (end 182.17 212.6452) (width 2) (layer "B.Cu") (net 30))
 (segment (start 182.17 212.6452) (end 182.2248 212.7) (width 2) (layer "B.Cu") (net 30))
 (segment (start 225.73 212.6188) (end 225.8112 212.7) (width 2) (layer "B.Cu") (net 19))
 (segment (start 225.73 23.82) (end 225.73 212.6188) (width 2) (layer "B.Cu") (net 19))
 (segment (start 229.69 23.82) (end 229.69 212.6164) (width 2) (layer "B.Cu") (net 18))
 (segment (start 229.69 212.6164) (end 229.7736 212.7) (width 2) (layer "B.Cu") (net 18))
 (segment (start 233.65 23.82) (end 233.65 212.614) (width 2) (layer "B.Cu") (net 17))
 (segment (start 233.65 212.614) (end 233.736 212.7) (width 2) (layer "B.Cu") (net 17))
 (segment (start 237.61 212.6116) (end 237.6984 212.7) (width 2) (layer "B.Cu") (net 16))
 (segment (start 237.61 23.82) (end 237.61 212.6116) (width 2) (layer "B.Cu") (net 16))
 (segment (start 241.57 212.6092) (end 241.6608 212.7) (width 2) (layer "B.Cu") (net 15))
 (segment (start 241.57 23.82) (end 241.57 212.6092) (width 2) (layer "B.Cu") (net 15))
 (segment (start 245.53 23.82) (end 245.53 212.6068) (width 2) (layer "B.Cu") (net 14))
 (segment (start 245.53 212.6068) (end 245.6232 212.7) (width 2) (layer "B.Cu") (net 14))
 (segment (start 249.49 212.6044) (end 249.5856 212.7) (width 2) (layer "B.Cu") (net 13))
 (segment (start 249.49 23.82) (end 249.49 212.6044) (width 2) (layer "B.Cu") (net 13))
 (segment (start 253.45 212.602) (end 253.548 212.7) (width 2) (layer "B.Cu") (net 12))
 (segment (start 253.45 23.82) (end 253.45 212.602) (width 2) (layer "B.Cu") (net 12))
 (segment (start 257.41 23.82) (end 257.41 212.5996) (width 2) (layer "B.Cu") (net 11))
 (segment (start 257.41 212.5996) (end 257.5104 212.7) (width 2) (layer "B.Cu") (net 11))
 (segment (start 261.37 23.82) (end 261.37 212.5972) (width 2) (layer "B.Cu") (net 10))
 (segment (start 261.37 212.5972) (end 261.4728 212.7) (width 2) (layer "B.Cu") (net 10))
 (segment (start 265.33 212.5948) (end 265.4352 212.7) (width 2) (layer "B.Cu") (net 9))
 (segment (start 265.33 23.82) (end 265.33 212.5948) (width 2) (layer "B.Cu") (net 9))
 (segment (start 269.29 23.82) (end 269.29 212.5924) (width 2) (layer "B.Cu") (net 8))
 (segment (start 269.29 212.5924) (end 269.3976 212.7) (width 2) (layer "B.Cu") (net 8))
 (segment (start 273.25 23.82) (end 273.25 212.59) (width 2) (layer "B.Cu") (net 7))
 (segment (start 273.25 212.59) (end 273.36 212.7) (width 2) (layer "B.Cu") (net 7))
 (segment (start 277.21 212.5876) (end 277.3224 212.7) (width 2) (layer "B.Cu") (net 6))
 (segment (start 277.21 23.82) (end 277.21 212.5876) (width 2) (layer "B.Cu") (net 6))
 (segment (start 281.17 23.82) (end 281.17 212.5852) (width 2) (layer "B.Cu") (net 5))
 (segment (start 281.17 212.5852) (end 281.2848 212.7) (width 2) (layer "B.Cu") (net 5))
 (segment (start 285.13 23.82) (end 285.13 212.5828) (width 2) (layer "B.Cu") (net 4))
 (segment (start 285.13 212.5828) (end 285.2472 212.7) (width 2) (layer "B.Cu") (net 4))
 (segment (start 289.09 23.82) (end 289.09 212.5804) (width 2) (layer "B.Cu") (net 3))
 (segment (start 289.09 212.5804) (end 289.2096 212.7) (width 2) (layer "B.Cu") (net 3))
 (segment (start 293.05 212.578) (end 293.172 212.7) (width 2) (layer "B.Cu") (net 2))
 (segment (start 293.05 23.82) (end 293.05 212.578) (width 2) (layer "B.Cu") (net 2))
 (segment (start 297.01 212.5756) (end 297.1344 212.7) (width 2) (layer "B.Cu") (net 1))
 (segment (start 297.01 23.82) (end 297.01 212.5756) (width 2) (layer "B.Cu") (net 1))
 (segment (start 85.15 212.7748) (end 85.1248 212.8) (width 2) (layer "B.Cu") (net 48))
 (segment (start 85.15 23.81) (end 85.15 212.7748) (width 2) (layer "B.Cu") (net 48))
 (segment (start 89.0872 23.8328) (end 89.11 23.81) (width 2) (layer "B.Cu") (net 47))
 (segment (start 89.0872 212.8) (end 89.0872 23.8328) (width 2) (layer "B.Cu") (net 47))
 (segment (start 89.11 23.81) (end 89.11 43.81) (width 2) (layer "B.Cu") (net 47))
 (segment (start 93.07 23.81) (end 93.07 211.87) (width 2) (layer "B.Cu") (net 46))
 (segment (start 97.03 23.81) (end 97.03 43.81) (width 2) (layer "B.Cu") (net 45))
 (segment (start 97.012 23.828) (end 97.03 23.81) (width 2) (layer "B.Cu") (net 45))
 (segment (start 97.012 212.8) (end 97.012 23.828) (width 2) (layer "B.Cu") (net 45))
 (segment (start 100.99 23.81) (end 100.99 212.7844) (width 2) (layer "B.Cu") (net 44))
 (segment (start 100.99 212.7844) (end 100.9744 212.8) (width 2) (layer "B.Cu") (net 44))
 (segment (start 104.95 212.7868) (end 104.9368 212.8) (width 2) (layer "B.Cu") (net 43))
 (segment (start 104.95 23.81) (end 104.95 212.7868) (width 2) (layer "B.Cu") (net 43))
 (segment (start 108.91 212.7892) (end 108.8992 212.8) (width 2) (layer "B.Cu") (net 42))
 (segment (start 108.91 23.81) (end 108.91 212.7892) (width 2) (layer "B.Cu") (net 42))
 (segment (start 112.87 212.7916) (end 112.8616 212.8) (width 2) (layer "B.Cu") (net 41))
 (segment (start 112.87 23.81) (end 112.87 212.7916) (width 2) (layer "B.Cu") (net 41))
 (segment (start 116.83 212.794) (end 116.824 212.8) (width 2) (layer "B.Cu") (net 40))
 (segment (start 116.83 23.81) (end 116.83 212.794) (width 2) (layer "B.Cu") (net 40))
 (segment (start 120.79 212.7964) (end 120.7864 212.8) (width 2) (layer "B.Cu") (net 39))
 (segment (start 120.79 23.81) (end 120.79 212.7964) (width 2) (layer "B.Cu") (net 39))
 (segment (start 124.75 212.7988) (end 124.7488 212.8) (width 2) (layer "B.Cu") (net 38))
 (segment (start 124.75 23.81) (end 124.75 212.7988) (width 2) (layer "B.Cu") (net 38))
 (segment (start 128.71 212.7988) (end 128.7112 212.8) (width 2) (layer "B.Cu") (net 37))
 (segment (start 128.71 23.81) (end 128.71 212.7988) (width 2) (layer "B.Cu") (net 37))
 (segment (start 132.67 23.81) (end 132.67 212.7964) (width 2) (layer "B.Cu") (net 36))
 (segment (start 132.67 212.7964) (end 132.6736 212.8) (width 2) (layer "B.Cu") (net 36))
 (segment (start 136.63 212.794) (end 136.636 212.8) (width 2) (layer "B.Cu") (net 35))
 (segment (start 136.63 23.81) (end 136.63 212.794) (width 2) (layer "B.Cu") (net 35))
 (segment (start 140.59 23.81) (end 140.59 212.7916) (width 2) (layer "B.Cu") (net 34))
 (segment (start 140.59 212.7916) (end 140.5984 212.8) (width 2) (layer "B.Cu") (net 34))
 (segment (start 144.55 212.7892) (end 144.5608 212.8) (width 2) (layer "B.Cu") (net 33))
 (segment (start 144.55 23.81) (end 144.55 212.7892) (width 2) (layer "B.Cu") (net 33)))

